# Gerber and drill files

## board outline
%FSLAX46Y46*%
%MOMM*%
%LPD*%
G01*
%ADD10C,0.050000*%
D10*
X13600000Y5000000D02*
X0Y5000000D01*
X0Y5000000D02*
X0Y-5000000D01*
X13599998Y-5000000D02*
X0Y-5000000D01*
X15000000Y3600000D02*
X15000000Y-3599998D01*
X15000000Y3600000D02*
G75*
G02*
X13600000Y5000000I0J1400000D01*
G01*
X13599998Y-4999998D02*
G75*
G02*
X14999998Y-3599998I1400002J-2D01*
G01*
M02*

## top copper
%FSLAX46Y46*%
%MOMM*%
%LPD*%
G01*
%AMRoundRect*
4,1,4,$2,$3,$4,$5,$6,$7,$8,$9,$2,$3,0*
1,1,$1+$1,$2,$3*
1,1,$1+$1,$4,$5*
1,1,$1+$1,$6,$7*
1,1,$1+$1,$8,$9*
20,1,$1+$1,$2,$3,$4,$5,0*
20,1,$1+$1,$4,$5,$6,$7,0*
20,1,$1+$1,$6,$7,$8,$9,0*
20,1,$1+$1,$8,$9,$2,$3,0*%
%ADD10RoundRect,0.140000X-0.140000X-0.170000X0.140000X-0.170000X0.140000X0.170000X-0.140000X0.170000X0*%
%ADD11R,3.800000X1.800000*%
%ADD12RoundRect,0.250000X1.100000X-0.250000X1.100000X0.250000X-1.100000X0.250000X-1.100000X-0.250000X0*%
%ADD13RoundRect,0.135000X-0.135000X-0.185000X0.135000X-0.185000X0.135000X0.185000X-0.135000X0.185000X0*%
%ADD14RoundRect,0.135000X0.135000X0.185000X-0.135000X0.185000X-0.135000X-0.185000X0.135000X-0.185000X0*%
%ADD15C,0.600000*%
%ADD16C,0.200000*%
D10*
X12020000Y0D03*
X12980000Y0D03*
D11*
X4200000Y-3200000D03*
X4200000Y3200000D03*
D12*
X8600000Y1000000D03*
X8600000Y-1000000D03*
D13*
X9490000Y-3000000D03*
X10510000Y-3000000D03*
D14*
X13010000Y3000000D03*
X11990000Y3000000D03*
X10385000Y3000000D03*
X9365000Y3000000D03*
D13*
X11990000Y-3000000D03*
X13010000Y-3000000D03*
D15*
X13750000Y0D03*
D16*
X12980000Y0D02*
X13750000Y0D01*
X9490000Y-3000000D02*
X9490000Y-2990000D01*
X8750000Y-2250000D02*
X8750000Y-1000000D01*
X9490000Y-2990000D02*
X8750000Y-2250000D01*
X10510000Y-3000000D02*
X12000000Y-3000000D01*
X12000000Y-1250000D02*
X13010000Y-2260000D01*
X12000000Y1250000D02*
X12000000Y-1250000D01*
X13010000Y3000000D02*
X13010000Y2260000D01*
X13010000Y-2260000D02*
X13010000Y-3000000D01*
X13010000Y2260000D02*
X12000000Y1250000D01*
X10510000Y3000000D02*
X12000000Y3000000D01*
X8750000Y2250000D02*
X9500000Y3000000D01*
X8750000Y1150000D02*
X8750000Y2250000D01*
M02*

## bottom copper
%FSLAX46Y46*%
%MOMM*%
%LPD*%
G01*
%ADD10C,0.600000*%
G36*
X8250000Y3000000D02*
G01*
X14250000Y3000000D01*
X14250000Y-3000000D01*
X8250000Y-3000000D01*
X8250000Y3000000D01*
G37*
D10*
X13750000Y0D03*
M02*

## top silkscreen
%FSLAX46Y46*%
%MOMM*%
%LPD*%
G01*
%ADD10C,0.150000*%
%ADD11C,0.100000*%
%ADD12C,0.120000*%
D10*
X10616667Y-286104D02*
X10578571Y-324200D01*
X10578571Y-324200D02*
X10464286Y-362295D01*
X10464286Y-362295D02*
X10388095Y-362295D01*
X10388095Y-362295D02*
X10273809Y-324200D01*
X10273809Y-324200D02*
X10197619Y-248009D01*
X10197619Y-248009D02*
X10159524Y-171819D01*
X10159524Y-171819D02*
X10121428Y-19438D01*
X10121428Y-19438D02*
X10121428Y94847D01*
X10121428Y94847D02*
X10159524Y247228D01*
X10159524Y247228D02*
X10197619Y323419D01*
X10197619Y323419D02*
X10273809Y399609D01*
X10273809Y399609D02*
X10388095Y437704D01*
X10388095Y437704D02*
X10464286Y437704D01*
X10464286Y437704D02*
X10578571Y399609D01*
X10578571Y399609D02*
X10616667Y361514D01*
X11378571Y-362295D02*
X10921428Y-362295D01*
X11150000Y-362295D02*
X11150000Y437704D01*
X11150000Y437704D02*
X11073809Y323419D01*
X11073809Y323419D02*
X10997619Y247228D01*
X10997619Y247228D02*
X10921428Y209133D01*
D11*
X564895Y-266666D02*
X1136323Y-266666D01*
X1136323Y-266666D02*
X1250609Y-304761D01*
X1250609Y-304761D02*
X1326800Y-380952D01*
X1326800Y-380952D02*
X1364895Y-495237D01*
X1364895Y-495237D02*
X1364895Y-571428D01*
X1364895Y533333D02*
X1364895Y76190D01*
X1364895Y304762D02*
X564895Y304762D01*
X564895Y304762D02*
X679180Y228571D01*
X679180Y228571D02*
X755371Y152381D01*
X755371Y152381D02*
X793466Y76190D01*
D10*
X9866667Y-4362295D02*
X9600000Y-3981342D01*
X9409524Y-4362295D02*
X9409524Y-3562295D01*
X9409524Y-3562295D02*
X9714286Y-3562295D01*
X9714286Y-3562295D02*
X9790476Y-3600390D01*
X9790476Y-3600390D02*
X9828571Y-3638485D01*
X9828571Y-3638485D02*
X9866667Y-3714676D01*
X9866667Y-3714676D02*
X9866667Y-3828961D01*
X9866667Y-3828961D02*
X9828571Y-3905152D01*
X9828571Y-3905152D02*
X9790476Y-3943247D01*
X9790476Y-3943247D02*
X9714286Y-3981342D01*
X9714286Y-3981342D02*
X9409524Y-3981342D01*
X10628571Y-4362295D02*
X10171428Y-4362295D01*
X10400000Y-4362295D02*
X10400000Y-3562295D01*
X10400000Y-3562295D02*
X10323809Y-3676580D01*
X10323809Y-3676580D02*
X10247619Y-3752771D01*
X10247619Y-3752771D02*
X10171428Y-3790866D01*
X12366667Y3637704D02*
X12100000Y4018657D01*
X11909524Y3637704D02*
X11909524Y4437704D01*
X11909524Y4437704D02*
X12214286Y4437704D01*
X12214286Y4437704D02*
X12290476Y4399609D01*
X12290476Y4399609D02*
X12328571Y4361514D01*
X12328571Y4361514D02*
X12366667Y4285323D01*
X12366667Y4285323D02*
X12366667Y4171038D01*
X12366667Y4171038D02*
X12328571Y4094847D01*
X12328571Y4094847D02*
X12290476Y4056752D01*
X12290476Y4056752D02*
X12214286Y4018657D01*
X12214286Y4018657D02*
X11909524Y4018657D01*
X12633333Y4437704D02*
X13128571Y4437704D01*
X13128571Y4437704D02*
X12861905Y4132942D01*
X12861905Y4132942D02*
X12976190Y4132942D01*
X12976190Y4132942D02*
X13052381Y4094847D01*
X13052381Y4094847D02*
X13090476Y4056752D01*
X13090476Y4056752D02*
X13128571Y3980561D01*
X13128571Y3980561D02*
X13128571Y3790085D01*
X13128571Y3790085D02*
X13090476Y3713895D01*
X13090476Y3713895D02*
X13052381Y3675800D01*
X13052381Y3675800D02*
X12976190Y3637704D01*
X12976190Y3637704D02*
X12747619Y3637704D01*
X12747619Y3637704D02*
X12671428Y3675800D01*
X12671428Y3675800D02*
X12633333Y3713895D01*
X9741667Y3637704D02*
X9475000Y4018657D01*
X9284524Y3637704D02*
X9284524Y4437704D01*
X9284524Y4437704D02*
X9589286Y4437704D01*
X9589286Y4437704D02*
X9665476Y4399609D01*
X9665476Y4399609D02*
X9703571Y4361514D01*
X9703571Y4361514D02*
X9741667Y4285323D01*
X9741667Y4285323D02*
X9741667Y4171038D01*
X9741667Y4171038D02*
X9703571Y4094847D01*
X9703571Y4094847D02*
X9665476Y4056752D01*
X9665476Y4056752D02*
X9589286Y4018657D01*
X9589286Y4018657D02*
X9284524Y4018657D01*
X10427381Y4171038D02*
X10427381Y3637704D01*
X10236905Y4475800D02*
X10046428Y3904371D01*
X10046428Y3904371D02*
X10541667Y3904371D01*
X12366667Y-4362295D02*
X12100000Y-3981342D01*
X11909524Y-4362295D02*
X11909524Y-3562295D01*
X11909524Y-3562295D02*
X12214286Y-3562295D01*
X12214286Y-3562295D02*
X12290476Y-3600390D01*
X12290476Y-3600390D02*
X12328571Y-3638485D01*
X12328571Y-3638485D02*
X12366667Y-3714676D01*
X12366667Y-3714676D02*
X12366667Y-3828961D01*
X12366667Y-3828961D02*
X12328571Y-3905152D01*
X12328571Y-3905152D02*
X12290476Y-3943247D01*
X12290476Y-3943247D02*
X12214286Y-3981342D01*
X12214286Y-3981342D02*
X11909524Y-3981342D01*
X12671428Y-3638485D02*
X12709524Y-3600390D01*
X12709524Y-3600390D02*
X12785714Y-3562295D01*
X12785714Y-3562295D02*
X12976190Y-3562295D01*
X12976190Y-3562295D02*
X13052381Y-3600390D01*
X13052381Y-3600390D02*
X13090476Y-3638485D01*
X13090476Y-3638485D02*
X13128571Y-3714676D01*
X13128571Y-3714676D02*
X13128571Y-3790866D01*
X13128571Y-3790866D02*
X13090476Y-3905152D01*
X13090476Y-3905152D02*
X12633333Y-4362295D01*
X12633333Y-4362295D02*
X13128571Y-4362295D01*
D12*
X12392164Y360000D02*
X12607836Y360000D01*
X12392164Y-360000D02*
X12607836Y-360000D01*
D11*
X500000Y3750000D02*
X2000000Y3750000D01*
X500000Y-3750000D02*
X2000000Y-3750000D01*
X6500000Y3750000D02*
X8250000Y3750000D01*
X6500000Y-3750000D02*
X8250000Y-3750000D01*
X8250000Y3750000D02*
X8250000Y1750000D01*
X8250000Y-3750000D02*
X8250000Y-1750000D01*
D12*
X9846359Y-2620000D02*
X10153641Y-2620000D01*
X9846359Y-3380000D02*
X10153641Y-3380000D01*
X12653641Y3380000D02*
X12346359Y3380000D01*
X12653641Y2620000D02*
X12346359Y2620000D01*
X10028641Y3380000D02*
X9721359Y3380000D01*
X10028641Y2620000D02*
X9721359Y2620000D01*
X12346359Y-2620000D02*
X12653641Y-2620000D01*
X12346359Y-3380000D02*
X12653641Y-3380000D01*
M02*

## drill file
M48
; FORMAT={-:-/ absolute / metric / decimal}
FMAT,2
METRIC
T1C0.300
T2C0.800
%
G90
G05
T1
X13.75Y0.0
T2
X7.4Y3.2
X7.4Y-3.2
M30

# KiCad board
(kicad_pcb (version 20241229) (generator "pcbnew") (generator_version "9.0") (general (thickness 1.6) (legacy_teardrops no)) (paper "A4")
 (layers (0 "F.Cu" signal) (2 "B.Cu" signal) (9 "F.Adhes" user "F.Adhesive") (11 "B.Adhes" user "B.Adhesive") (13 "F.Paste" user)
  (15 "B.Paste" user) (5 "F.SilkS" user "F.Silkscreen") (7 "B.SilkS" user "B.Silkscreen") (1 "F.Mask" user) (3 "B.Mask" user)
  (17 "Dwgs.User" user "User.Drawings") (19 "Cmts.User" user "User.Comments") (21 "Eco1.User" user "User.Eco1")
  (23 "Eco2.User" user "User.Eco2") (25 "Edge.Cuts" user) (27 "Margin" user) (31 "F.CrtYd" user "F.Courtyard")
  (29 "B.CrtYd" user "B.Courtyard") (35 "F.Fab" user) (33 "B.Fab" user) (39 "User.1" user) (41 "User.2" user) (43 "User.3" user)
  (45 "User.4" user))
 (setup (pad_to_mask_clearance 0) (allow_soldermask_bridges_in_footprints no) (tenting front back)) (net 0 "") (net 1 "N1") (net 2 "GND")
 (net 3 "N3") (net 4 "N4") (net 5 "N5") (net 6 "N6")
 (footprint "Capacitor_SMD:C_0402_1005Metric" (layer "F.Cu") (at 12.5 0)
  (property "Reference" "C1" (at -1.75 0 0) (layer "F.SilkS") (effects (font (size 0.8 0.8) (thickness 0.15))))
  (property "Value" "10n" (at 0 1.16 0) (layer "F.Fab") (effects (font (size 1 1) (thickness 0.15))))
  (fp_line (start -0.107836 -0.36) (end 0.107836 -0.36) (stroke (width 0.12) (type solid)) (layer "F.SilkS"))
  (fp_line (start -0.107836 0.36) (end 0.107836 0.36) (stroke (width 0.12) (type solid)) (layer "F.SilkS"))
  (pad "1" smd roundrect (at -0.48 0) (size 0.56 0.62) (layers "F.Cu" "F.Mask" "F.Paste") (roundrect_rratio 0.25) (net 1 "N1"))
  (pad "2" smd roundrect (at 0.48 0) (size 0.56 0.62) (layers "F.Cu" "F.Mask" "F.Paste") (roundrect_rratio 0.25) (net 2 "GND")))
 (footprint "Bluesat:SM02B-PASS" (layer "F.Cu") (at 0 0 90)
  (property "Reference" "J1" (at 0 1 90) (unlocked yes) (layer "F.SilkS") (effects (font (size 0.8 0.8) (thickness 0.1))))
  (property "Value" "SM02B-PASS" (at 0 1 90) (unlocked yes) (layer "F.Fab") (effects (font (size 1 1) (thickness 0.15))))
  (fp_line (start 3.75 0.5) (end 3.75 2) (stroke (width 0.1) (type default)) (layer "F.SilkS"))
  (fp_line (start -3.75 0.5) (end -3.75 2) (stroke (width 0.1) (type default)) (layer "F.SilkS"))
  (fp_line (start 3.75 6.5) (end 3.75 8.25) (stroke (width 0.1) (type default)) (layer "F.SilkS"))
  (fp_line (start -3.75 6.5) (end -3.75 8.25) (stroke (width 0.1) (type default)) (layer "F.SilkS"))
  (fp_line (start 3.75 8.25) (end 1.75 8.25) (stroke (width 0.1) (type default)) (layer "F.SilkS"))
  (fp_line (start -3.75 8.25) (end -1.75 8.25) (stroke (width 0.1) (type default)) (layer "F.SilkS"))
  (pad "" smd rect (at -3.2 4.2 90) (size 1.8 3.8) (layers "F.Cu" "F.Mask" "F.Paste") (thermal_bridge_angle 45))
  (pad "" np_thru_hole circle (at -3.2 7.4 90) (size 0.8 0.8) (drill 0.8) (layers "*.Mask"))
  (pad "" smd rect (at 3.2 4.2 90) (size 1.8 3.8) (layers "F.Cu" "F.Mask" "F.Paste") (thermal_bridge_angle 45))
  (pad "" np_thru_hole circle (at 3.2 7.4 90) (size 0.8 0.8) (drill 0.8) (layers "*.Mask"))
  (pad "1" smd roundrect (at 1 8.6 90) (size 1 2.7) (layers "F.Cu" "F.Mask" "F.Paste") (roundrect_rratio 0.25) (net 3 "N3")
   (thermal_bridge_angle 45))
  (pad "2" smd roundrect (at -1 8.6 90) (size 1 2.7) (layers "F.Cu" "F.Mask" "F.Paste") (roundrect_rratio 0.25) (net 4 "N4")
   (thermal_bridge_angle 45)))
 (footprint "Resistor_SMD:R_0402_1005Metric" (layer "F.Cu") (at 10 3)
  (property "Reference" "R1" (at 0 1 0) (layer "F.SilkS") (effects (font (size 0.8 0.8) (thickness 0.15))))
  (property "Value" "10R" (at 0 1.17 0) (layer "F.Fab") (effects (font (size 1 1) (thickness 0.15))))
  (fp_line (start -0.153641 -0.38) (end 0.153641 -0.38) (stroke (width 0.12) (type solid)) (layer "F.SilkS"))
  (fp_line (start -0.153641 0.38) (end 0.153641 0.38) (stroke (width 0.12) (type solid)) (layer "F.SilkS"))
  (pad "1" smd roundrect (at -0.51 0) (size 0.54 0.64) (layers "F.Cu" "F.Mask" "F.Paste") (roundrect_rratio 0.25) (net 4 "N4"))
  (pad "2" smd roundrect (at 0.51 0) (size 0.54 0.64) (layers "F.Cu" "F.Mask" "F.Paste") (roundrect_rratio 0.25) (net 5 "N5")))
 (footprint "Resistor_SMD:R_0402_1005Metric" (layer "F.Cu") (at 12.5 -3 180)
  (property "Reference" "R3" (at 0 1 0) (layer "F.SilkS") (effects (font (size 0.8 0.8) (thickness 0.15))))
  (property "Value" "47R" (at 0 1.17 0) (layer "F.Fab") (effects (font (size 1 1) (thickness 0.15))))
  (fp_line (start -0.153641 0.38) (end 0.153641 0.38) (stroke (width 0.12) (type solid)) (layer "F.SilkS"))
  (fp_line (start -0.153641 -0.38) (end 0.153641 -0.38) (stroke (width 0.12) (type solid)) (layer "F.SilkS"))
  (pad "1" smd roundrect (at -0.51 0 180) (size 0.54 0.64) (layers "F.Cu" "F.Mask" "F.Paste") (roundrect_rratio 0.25) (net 1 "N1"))
  (pad "2" smd roundrect (at 0.51 0 180) (size 0.54 0.64) (layers "F.Cu" "F.Mask" "F.Paste") (roundrect_rratio 0.25) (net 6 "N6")))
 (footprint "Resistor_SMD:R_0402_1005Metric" (layer "F.Cu") (at 9.875 -3 180)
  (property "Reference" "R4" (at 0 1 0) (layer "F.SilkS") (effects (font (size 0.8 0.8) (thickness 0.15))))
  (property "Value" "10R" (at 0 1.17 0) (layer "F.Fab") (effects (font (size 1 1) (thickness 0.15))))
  (fp_line (start -0.153641 0.38) (end 0.153641 0.38) (stroke (width 0.12) (type solid)) (layer "F.SilkS"))
  (fp_line (start -0.153641 -0.38) (end 0.153641 -0.38) (stroke (width 0.12) (type solid)) (layer "F.SilkS"))
  (pad "1" smd roundrect (at -0.51 0 180) (size 0.54 0.64) (layers "F.Cu" "F.Mask" "F.Paste") (roundrect_rratio 0.25) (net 6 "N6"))
  (pad "2" smd roundrect (at 0.51 0 180) (size 0.54 0.64) (layers "F.Cu" "F.Mask" "F.Paste") (roundrect_rratio 0.25) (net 3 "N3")))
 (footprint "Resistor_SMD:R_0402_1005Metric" (layer "F.Cu") (at 12.5 3)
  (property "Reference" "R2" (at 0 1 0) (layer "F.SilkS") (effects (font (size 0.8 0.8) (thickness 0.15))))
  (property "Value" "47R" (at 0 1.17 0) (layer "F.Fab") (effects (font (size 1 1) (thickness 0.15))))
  (fp_line (start -0.153641 -0.38) (end 0.153641 -0.38) (stroke (width 0.12) (type solid)) (layer "F.SilkS"))
  (fp_line (start -0.153641 0.38) (end 0.153641 0.38) (stroke (width 0.12) (type solid)) (layer "F.SilkS"))
  (pad "1" smd roundrect (at -0.51 0) (size 0.54 0.64) (layers "F.Cu" "F.Mask" "F.Paste") (roundrect_rratio 0.25) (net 5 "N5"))
  (pad "2" smd roundrect (at 0.51 0) (size 0.54 0.64) (layers "F.Cu" "F.Mask" "F.Paste") (roundrect_rratio 0.25) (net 1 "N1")))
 (gr_rect (start 8.25 -3) (end 14.25 3) (stroke (width 0) (type solid)) (fill yes) (layers "B.Cu" "B.Mask") (net 2))
 (gr_line (start 13.6 -5) (end 0 -5) (stroke (width 0.05) (type default)) (layer "Edge.Cuts"))
 (gr_line (start 0 -5) (end 0 5) (stroke (width 0.05) (type default)) (layer "Edge.Cuts"))
 (gr_line (start 13.599998 5) (end 0 5) (stroke (width 0.05) (type default)) (layer "Edge.Cuts"))
 (gr_line (start 15 -3.6) (end 15 3.599998) (stroke (width 0.05) (type default)) (layer "Edge.Cuts"))
 (gr_arc (start 15 -3.6) (mid 14.010051 -4.010051) (end 13.6 -5) (stroke (width 0.05) (type solid)) (layer "Edge.Cuts"))
 (gr_arc (start 13.599998 4.999998) (mid 14.010049 4.010049) (end 14.999998 3.599998) (stroke (width 0.05) (type solid)) (layer "Edge.Cuts"))
 (segment (start 12.98 0) (end 13.75 0) (width 0.2) (layer "F.Cu") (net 2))
 (via (at 13.75 0) (size 0.6) (drill 0.3) (layers "F.Cu" "B.Cu") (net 2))
 (segment (start 9.49 3) (end 9.49 2.99) (width 0.2) (layer "F.Cu") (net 4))
 (segment (start 8.75 2.25) (end 8.75 1) (width 0.2) (layer "F.Cu") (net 4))
 (segment (start 9.49 2.99) (end 8.75 2.25) (width 0.2) (layer "F.Cu") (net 4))
 (segment (start 10.51 3) (end 12 3) (width 0.2) (layer "F.Cu") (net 5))
 (segment (start 12 1.25) (end 13.01 2.26) (width 0.2) (layer "F.Cu") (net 1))
 (segment (start 12 -1.25) (end 12 1.25) (width 0.2) (layer "F.Cu") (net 1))
 (segment (start 13.01 -3) (end 13.01 -2.26) (width 0.2) (layer "F.Cu") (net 1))
 (segment (start 13.01 2.26) (end 13.01 3) (width 0.2) (layer "F.Cu") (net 1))
 (segment (start 13.01 -2.26) (end 12 -1.25) (width 0.2) (layer "F.Cu") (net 1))
 (segment (start 10.51 -3) (end 12 -3) (width 0.2) (layer "F.Cu") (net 6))
 (segment (start 8.75 -2.25) (end 9.5 -3) (width 0.2) (layer "F.Cu") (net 3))
 (segment (start 8.75 -1.15) (end 8.75 -2.25) (width 0.2) (layer "F.Cu") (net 3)))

